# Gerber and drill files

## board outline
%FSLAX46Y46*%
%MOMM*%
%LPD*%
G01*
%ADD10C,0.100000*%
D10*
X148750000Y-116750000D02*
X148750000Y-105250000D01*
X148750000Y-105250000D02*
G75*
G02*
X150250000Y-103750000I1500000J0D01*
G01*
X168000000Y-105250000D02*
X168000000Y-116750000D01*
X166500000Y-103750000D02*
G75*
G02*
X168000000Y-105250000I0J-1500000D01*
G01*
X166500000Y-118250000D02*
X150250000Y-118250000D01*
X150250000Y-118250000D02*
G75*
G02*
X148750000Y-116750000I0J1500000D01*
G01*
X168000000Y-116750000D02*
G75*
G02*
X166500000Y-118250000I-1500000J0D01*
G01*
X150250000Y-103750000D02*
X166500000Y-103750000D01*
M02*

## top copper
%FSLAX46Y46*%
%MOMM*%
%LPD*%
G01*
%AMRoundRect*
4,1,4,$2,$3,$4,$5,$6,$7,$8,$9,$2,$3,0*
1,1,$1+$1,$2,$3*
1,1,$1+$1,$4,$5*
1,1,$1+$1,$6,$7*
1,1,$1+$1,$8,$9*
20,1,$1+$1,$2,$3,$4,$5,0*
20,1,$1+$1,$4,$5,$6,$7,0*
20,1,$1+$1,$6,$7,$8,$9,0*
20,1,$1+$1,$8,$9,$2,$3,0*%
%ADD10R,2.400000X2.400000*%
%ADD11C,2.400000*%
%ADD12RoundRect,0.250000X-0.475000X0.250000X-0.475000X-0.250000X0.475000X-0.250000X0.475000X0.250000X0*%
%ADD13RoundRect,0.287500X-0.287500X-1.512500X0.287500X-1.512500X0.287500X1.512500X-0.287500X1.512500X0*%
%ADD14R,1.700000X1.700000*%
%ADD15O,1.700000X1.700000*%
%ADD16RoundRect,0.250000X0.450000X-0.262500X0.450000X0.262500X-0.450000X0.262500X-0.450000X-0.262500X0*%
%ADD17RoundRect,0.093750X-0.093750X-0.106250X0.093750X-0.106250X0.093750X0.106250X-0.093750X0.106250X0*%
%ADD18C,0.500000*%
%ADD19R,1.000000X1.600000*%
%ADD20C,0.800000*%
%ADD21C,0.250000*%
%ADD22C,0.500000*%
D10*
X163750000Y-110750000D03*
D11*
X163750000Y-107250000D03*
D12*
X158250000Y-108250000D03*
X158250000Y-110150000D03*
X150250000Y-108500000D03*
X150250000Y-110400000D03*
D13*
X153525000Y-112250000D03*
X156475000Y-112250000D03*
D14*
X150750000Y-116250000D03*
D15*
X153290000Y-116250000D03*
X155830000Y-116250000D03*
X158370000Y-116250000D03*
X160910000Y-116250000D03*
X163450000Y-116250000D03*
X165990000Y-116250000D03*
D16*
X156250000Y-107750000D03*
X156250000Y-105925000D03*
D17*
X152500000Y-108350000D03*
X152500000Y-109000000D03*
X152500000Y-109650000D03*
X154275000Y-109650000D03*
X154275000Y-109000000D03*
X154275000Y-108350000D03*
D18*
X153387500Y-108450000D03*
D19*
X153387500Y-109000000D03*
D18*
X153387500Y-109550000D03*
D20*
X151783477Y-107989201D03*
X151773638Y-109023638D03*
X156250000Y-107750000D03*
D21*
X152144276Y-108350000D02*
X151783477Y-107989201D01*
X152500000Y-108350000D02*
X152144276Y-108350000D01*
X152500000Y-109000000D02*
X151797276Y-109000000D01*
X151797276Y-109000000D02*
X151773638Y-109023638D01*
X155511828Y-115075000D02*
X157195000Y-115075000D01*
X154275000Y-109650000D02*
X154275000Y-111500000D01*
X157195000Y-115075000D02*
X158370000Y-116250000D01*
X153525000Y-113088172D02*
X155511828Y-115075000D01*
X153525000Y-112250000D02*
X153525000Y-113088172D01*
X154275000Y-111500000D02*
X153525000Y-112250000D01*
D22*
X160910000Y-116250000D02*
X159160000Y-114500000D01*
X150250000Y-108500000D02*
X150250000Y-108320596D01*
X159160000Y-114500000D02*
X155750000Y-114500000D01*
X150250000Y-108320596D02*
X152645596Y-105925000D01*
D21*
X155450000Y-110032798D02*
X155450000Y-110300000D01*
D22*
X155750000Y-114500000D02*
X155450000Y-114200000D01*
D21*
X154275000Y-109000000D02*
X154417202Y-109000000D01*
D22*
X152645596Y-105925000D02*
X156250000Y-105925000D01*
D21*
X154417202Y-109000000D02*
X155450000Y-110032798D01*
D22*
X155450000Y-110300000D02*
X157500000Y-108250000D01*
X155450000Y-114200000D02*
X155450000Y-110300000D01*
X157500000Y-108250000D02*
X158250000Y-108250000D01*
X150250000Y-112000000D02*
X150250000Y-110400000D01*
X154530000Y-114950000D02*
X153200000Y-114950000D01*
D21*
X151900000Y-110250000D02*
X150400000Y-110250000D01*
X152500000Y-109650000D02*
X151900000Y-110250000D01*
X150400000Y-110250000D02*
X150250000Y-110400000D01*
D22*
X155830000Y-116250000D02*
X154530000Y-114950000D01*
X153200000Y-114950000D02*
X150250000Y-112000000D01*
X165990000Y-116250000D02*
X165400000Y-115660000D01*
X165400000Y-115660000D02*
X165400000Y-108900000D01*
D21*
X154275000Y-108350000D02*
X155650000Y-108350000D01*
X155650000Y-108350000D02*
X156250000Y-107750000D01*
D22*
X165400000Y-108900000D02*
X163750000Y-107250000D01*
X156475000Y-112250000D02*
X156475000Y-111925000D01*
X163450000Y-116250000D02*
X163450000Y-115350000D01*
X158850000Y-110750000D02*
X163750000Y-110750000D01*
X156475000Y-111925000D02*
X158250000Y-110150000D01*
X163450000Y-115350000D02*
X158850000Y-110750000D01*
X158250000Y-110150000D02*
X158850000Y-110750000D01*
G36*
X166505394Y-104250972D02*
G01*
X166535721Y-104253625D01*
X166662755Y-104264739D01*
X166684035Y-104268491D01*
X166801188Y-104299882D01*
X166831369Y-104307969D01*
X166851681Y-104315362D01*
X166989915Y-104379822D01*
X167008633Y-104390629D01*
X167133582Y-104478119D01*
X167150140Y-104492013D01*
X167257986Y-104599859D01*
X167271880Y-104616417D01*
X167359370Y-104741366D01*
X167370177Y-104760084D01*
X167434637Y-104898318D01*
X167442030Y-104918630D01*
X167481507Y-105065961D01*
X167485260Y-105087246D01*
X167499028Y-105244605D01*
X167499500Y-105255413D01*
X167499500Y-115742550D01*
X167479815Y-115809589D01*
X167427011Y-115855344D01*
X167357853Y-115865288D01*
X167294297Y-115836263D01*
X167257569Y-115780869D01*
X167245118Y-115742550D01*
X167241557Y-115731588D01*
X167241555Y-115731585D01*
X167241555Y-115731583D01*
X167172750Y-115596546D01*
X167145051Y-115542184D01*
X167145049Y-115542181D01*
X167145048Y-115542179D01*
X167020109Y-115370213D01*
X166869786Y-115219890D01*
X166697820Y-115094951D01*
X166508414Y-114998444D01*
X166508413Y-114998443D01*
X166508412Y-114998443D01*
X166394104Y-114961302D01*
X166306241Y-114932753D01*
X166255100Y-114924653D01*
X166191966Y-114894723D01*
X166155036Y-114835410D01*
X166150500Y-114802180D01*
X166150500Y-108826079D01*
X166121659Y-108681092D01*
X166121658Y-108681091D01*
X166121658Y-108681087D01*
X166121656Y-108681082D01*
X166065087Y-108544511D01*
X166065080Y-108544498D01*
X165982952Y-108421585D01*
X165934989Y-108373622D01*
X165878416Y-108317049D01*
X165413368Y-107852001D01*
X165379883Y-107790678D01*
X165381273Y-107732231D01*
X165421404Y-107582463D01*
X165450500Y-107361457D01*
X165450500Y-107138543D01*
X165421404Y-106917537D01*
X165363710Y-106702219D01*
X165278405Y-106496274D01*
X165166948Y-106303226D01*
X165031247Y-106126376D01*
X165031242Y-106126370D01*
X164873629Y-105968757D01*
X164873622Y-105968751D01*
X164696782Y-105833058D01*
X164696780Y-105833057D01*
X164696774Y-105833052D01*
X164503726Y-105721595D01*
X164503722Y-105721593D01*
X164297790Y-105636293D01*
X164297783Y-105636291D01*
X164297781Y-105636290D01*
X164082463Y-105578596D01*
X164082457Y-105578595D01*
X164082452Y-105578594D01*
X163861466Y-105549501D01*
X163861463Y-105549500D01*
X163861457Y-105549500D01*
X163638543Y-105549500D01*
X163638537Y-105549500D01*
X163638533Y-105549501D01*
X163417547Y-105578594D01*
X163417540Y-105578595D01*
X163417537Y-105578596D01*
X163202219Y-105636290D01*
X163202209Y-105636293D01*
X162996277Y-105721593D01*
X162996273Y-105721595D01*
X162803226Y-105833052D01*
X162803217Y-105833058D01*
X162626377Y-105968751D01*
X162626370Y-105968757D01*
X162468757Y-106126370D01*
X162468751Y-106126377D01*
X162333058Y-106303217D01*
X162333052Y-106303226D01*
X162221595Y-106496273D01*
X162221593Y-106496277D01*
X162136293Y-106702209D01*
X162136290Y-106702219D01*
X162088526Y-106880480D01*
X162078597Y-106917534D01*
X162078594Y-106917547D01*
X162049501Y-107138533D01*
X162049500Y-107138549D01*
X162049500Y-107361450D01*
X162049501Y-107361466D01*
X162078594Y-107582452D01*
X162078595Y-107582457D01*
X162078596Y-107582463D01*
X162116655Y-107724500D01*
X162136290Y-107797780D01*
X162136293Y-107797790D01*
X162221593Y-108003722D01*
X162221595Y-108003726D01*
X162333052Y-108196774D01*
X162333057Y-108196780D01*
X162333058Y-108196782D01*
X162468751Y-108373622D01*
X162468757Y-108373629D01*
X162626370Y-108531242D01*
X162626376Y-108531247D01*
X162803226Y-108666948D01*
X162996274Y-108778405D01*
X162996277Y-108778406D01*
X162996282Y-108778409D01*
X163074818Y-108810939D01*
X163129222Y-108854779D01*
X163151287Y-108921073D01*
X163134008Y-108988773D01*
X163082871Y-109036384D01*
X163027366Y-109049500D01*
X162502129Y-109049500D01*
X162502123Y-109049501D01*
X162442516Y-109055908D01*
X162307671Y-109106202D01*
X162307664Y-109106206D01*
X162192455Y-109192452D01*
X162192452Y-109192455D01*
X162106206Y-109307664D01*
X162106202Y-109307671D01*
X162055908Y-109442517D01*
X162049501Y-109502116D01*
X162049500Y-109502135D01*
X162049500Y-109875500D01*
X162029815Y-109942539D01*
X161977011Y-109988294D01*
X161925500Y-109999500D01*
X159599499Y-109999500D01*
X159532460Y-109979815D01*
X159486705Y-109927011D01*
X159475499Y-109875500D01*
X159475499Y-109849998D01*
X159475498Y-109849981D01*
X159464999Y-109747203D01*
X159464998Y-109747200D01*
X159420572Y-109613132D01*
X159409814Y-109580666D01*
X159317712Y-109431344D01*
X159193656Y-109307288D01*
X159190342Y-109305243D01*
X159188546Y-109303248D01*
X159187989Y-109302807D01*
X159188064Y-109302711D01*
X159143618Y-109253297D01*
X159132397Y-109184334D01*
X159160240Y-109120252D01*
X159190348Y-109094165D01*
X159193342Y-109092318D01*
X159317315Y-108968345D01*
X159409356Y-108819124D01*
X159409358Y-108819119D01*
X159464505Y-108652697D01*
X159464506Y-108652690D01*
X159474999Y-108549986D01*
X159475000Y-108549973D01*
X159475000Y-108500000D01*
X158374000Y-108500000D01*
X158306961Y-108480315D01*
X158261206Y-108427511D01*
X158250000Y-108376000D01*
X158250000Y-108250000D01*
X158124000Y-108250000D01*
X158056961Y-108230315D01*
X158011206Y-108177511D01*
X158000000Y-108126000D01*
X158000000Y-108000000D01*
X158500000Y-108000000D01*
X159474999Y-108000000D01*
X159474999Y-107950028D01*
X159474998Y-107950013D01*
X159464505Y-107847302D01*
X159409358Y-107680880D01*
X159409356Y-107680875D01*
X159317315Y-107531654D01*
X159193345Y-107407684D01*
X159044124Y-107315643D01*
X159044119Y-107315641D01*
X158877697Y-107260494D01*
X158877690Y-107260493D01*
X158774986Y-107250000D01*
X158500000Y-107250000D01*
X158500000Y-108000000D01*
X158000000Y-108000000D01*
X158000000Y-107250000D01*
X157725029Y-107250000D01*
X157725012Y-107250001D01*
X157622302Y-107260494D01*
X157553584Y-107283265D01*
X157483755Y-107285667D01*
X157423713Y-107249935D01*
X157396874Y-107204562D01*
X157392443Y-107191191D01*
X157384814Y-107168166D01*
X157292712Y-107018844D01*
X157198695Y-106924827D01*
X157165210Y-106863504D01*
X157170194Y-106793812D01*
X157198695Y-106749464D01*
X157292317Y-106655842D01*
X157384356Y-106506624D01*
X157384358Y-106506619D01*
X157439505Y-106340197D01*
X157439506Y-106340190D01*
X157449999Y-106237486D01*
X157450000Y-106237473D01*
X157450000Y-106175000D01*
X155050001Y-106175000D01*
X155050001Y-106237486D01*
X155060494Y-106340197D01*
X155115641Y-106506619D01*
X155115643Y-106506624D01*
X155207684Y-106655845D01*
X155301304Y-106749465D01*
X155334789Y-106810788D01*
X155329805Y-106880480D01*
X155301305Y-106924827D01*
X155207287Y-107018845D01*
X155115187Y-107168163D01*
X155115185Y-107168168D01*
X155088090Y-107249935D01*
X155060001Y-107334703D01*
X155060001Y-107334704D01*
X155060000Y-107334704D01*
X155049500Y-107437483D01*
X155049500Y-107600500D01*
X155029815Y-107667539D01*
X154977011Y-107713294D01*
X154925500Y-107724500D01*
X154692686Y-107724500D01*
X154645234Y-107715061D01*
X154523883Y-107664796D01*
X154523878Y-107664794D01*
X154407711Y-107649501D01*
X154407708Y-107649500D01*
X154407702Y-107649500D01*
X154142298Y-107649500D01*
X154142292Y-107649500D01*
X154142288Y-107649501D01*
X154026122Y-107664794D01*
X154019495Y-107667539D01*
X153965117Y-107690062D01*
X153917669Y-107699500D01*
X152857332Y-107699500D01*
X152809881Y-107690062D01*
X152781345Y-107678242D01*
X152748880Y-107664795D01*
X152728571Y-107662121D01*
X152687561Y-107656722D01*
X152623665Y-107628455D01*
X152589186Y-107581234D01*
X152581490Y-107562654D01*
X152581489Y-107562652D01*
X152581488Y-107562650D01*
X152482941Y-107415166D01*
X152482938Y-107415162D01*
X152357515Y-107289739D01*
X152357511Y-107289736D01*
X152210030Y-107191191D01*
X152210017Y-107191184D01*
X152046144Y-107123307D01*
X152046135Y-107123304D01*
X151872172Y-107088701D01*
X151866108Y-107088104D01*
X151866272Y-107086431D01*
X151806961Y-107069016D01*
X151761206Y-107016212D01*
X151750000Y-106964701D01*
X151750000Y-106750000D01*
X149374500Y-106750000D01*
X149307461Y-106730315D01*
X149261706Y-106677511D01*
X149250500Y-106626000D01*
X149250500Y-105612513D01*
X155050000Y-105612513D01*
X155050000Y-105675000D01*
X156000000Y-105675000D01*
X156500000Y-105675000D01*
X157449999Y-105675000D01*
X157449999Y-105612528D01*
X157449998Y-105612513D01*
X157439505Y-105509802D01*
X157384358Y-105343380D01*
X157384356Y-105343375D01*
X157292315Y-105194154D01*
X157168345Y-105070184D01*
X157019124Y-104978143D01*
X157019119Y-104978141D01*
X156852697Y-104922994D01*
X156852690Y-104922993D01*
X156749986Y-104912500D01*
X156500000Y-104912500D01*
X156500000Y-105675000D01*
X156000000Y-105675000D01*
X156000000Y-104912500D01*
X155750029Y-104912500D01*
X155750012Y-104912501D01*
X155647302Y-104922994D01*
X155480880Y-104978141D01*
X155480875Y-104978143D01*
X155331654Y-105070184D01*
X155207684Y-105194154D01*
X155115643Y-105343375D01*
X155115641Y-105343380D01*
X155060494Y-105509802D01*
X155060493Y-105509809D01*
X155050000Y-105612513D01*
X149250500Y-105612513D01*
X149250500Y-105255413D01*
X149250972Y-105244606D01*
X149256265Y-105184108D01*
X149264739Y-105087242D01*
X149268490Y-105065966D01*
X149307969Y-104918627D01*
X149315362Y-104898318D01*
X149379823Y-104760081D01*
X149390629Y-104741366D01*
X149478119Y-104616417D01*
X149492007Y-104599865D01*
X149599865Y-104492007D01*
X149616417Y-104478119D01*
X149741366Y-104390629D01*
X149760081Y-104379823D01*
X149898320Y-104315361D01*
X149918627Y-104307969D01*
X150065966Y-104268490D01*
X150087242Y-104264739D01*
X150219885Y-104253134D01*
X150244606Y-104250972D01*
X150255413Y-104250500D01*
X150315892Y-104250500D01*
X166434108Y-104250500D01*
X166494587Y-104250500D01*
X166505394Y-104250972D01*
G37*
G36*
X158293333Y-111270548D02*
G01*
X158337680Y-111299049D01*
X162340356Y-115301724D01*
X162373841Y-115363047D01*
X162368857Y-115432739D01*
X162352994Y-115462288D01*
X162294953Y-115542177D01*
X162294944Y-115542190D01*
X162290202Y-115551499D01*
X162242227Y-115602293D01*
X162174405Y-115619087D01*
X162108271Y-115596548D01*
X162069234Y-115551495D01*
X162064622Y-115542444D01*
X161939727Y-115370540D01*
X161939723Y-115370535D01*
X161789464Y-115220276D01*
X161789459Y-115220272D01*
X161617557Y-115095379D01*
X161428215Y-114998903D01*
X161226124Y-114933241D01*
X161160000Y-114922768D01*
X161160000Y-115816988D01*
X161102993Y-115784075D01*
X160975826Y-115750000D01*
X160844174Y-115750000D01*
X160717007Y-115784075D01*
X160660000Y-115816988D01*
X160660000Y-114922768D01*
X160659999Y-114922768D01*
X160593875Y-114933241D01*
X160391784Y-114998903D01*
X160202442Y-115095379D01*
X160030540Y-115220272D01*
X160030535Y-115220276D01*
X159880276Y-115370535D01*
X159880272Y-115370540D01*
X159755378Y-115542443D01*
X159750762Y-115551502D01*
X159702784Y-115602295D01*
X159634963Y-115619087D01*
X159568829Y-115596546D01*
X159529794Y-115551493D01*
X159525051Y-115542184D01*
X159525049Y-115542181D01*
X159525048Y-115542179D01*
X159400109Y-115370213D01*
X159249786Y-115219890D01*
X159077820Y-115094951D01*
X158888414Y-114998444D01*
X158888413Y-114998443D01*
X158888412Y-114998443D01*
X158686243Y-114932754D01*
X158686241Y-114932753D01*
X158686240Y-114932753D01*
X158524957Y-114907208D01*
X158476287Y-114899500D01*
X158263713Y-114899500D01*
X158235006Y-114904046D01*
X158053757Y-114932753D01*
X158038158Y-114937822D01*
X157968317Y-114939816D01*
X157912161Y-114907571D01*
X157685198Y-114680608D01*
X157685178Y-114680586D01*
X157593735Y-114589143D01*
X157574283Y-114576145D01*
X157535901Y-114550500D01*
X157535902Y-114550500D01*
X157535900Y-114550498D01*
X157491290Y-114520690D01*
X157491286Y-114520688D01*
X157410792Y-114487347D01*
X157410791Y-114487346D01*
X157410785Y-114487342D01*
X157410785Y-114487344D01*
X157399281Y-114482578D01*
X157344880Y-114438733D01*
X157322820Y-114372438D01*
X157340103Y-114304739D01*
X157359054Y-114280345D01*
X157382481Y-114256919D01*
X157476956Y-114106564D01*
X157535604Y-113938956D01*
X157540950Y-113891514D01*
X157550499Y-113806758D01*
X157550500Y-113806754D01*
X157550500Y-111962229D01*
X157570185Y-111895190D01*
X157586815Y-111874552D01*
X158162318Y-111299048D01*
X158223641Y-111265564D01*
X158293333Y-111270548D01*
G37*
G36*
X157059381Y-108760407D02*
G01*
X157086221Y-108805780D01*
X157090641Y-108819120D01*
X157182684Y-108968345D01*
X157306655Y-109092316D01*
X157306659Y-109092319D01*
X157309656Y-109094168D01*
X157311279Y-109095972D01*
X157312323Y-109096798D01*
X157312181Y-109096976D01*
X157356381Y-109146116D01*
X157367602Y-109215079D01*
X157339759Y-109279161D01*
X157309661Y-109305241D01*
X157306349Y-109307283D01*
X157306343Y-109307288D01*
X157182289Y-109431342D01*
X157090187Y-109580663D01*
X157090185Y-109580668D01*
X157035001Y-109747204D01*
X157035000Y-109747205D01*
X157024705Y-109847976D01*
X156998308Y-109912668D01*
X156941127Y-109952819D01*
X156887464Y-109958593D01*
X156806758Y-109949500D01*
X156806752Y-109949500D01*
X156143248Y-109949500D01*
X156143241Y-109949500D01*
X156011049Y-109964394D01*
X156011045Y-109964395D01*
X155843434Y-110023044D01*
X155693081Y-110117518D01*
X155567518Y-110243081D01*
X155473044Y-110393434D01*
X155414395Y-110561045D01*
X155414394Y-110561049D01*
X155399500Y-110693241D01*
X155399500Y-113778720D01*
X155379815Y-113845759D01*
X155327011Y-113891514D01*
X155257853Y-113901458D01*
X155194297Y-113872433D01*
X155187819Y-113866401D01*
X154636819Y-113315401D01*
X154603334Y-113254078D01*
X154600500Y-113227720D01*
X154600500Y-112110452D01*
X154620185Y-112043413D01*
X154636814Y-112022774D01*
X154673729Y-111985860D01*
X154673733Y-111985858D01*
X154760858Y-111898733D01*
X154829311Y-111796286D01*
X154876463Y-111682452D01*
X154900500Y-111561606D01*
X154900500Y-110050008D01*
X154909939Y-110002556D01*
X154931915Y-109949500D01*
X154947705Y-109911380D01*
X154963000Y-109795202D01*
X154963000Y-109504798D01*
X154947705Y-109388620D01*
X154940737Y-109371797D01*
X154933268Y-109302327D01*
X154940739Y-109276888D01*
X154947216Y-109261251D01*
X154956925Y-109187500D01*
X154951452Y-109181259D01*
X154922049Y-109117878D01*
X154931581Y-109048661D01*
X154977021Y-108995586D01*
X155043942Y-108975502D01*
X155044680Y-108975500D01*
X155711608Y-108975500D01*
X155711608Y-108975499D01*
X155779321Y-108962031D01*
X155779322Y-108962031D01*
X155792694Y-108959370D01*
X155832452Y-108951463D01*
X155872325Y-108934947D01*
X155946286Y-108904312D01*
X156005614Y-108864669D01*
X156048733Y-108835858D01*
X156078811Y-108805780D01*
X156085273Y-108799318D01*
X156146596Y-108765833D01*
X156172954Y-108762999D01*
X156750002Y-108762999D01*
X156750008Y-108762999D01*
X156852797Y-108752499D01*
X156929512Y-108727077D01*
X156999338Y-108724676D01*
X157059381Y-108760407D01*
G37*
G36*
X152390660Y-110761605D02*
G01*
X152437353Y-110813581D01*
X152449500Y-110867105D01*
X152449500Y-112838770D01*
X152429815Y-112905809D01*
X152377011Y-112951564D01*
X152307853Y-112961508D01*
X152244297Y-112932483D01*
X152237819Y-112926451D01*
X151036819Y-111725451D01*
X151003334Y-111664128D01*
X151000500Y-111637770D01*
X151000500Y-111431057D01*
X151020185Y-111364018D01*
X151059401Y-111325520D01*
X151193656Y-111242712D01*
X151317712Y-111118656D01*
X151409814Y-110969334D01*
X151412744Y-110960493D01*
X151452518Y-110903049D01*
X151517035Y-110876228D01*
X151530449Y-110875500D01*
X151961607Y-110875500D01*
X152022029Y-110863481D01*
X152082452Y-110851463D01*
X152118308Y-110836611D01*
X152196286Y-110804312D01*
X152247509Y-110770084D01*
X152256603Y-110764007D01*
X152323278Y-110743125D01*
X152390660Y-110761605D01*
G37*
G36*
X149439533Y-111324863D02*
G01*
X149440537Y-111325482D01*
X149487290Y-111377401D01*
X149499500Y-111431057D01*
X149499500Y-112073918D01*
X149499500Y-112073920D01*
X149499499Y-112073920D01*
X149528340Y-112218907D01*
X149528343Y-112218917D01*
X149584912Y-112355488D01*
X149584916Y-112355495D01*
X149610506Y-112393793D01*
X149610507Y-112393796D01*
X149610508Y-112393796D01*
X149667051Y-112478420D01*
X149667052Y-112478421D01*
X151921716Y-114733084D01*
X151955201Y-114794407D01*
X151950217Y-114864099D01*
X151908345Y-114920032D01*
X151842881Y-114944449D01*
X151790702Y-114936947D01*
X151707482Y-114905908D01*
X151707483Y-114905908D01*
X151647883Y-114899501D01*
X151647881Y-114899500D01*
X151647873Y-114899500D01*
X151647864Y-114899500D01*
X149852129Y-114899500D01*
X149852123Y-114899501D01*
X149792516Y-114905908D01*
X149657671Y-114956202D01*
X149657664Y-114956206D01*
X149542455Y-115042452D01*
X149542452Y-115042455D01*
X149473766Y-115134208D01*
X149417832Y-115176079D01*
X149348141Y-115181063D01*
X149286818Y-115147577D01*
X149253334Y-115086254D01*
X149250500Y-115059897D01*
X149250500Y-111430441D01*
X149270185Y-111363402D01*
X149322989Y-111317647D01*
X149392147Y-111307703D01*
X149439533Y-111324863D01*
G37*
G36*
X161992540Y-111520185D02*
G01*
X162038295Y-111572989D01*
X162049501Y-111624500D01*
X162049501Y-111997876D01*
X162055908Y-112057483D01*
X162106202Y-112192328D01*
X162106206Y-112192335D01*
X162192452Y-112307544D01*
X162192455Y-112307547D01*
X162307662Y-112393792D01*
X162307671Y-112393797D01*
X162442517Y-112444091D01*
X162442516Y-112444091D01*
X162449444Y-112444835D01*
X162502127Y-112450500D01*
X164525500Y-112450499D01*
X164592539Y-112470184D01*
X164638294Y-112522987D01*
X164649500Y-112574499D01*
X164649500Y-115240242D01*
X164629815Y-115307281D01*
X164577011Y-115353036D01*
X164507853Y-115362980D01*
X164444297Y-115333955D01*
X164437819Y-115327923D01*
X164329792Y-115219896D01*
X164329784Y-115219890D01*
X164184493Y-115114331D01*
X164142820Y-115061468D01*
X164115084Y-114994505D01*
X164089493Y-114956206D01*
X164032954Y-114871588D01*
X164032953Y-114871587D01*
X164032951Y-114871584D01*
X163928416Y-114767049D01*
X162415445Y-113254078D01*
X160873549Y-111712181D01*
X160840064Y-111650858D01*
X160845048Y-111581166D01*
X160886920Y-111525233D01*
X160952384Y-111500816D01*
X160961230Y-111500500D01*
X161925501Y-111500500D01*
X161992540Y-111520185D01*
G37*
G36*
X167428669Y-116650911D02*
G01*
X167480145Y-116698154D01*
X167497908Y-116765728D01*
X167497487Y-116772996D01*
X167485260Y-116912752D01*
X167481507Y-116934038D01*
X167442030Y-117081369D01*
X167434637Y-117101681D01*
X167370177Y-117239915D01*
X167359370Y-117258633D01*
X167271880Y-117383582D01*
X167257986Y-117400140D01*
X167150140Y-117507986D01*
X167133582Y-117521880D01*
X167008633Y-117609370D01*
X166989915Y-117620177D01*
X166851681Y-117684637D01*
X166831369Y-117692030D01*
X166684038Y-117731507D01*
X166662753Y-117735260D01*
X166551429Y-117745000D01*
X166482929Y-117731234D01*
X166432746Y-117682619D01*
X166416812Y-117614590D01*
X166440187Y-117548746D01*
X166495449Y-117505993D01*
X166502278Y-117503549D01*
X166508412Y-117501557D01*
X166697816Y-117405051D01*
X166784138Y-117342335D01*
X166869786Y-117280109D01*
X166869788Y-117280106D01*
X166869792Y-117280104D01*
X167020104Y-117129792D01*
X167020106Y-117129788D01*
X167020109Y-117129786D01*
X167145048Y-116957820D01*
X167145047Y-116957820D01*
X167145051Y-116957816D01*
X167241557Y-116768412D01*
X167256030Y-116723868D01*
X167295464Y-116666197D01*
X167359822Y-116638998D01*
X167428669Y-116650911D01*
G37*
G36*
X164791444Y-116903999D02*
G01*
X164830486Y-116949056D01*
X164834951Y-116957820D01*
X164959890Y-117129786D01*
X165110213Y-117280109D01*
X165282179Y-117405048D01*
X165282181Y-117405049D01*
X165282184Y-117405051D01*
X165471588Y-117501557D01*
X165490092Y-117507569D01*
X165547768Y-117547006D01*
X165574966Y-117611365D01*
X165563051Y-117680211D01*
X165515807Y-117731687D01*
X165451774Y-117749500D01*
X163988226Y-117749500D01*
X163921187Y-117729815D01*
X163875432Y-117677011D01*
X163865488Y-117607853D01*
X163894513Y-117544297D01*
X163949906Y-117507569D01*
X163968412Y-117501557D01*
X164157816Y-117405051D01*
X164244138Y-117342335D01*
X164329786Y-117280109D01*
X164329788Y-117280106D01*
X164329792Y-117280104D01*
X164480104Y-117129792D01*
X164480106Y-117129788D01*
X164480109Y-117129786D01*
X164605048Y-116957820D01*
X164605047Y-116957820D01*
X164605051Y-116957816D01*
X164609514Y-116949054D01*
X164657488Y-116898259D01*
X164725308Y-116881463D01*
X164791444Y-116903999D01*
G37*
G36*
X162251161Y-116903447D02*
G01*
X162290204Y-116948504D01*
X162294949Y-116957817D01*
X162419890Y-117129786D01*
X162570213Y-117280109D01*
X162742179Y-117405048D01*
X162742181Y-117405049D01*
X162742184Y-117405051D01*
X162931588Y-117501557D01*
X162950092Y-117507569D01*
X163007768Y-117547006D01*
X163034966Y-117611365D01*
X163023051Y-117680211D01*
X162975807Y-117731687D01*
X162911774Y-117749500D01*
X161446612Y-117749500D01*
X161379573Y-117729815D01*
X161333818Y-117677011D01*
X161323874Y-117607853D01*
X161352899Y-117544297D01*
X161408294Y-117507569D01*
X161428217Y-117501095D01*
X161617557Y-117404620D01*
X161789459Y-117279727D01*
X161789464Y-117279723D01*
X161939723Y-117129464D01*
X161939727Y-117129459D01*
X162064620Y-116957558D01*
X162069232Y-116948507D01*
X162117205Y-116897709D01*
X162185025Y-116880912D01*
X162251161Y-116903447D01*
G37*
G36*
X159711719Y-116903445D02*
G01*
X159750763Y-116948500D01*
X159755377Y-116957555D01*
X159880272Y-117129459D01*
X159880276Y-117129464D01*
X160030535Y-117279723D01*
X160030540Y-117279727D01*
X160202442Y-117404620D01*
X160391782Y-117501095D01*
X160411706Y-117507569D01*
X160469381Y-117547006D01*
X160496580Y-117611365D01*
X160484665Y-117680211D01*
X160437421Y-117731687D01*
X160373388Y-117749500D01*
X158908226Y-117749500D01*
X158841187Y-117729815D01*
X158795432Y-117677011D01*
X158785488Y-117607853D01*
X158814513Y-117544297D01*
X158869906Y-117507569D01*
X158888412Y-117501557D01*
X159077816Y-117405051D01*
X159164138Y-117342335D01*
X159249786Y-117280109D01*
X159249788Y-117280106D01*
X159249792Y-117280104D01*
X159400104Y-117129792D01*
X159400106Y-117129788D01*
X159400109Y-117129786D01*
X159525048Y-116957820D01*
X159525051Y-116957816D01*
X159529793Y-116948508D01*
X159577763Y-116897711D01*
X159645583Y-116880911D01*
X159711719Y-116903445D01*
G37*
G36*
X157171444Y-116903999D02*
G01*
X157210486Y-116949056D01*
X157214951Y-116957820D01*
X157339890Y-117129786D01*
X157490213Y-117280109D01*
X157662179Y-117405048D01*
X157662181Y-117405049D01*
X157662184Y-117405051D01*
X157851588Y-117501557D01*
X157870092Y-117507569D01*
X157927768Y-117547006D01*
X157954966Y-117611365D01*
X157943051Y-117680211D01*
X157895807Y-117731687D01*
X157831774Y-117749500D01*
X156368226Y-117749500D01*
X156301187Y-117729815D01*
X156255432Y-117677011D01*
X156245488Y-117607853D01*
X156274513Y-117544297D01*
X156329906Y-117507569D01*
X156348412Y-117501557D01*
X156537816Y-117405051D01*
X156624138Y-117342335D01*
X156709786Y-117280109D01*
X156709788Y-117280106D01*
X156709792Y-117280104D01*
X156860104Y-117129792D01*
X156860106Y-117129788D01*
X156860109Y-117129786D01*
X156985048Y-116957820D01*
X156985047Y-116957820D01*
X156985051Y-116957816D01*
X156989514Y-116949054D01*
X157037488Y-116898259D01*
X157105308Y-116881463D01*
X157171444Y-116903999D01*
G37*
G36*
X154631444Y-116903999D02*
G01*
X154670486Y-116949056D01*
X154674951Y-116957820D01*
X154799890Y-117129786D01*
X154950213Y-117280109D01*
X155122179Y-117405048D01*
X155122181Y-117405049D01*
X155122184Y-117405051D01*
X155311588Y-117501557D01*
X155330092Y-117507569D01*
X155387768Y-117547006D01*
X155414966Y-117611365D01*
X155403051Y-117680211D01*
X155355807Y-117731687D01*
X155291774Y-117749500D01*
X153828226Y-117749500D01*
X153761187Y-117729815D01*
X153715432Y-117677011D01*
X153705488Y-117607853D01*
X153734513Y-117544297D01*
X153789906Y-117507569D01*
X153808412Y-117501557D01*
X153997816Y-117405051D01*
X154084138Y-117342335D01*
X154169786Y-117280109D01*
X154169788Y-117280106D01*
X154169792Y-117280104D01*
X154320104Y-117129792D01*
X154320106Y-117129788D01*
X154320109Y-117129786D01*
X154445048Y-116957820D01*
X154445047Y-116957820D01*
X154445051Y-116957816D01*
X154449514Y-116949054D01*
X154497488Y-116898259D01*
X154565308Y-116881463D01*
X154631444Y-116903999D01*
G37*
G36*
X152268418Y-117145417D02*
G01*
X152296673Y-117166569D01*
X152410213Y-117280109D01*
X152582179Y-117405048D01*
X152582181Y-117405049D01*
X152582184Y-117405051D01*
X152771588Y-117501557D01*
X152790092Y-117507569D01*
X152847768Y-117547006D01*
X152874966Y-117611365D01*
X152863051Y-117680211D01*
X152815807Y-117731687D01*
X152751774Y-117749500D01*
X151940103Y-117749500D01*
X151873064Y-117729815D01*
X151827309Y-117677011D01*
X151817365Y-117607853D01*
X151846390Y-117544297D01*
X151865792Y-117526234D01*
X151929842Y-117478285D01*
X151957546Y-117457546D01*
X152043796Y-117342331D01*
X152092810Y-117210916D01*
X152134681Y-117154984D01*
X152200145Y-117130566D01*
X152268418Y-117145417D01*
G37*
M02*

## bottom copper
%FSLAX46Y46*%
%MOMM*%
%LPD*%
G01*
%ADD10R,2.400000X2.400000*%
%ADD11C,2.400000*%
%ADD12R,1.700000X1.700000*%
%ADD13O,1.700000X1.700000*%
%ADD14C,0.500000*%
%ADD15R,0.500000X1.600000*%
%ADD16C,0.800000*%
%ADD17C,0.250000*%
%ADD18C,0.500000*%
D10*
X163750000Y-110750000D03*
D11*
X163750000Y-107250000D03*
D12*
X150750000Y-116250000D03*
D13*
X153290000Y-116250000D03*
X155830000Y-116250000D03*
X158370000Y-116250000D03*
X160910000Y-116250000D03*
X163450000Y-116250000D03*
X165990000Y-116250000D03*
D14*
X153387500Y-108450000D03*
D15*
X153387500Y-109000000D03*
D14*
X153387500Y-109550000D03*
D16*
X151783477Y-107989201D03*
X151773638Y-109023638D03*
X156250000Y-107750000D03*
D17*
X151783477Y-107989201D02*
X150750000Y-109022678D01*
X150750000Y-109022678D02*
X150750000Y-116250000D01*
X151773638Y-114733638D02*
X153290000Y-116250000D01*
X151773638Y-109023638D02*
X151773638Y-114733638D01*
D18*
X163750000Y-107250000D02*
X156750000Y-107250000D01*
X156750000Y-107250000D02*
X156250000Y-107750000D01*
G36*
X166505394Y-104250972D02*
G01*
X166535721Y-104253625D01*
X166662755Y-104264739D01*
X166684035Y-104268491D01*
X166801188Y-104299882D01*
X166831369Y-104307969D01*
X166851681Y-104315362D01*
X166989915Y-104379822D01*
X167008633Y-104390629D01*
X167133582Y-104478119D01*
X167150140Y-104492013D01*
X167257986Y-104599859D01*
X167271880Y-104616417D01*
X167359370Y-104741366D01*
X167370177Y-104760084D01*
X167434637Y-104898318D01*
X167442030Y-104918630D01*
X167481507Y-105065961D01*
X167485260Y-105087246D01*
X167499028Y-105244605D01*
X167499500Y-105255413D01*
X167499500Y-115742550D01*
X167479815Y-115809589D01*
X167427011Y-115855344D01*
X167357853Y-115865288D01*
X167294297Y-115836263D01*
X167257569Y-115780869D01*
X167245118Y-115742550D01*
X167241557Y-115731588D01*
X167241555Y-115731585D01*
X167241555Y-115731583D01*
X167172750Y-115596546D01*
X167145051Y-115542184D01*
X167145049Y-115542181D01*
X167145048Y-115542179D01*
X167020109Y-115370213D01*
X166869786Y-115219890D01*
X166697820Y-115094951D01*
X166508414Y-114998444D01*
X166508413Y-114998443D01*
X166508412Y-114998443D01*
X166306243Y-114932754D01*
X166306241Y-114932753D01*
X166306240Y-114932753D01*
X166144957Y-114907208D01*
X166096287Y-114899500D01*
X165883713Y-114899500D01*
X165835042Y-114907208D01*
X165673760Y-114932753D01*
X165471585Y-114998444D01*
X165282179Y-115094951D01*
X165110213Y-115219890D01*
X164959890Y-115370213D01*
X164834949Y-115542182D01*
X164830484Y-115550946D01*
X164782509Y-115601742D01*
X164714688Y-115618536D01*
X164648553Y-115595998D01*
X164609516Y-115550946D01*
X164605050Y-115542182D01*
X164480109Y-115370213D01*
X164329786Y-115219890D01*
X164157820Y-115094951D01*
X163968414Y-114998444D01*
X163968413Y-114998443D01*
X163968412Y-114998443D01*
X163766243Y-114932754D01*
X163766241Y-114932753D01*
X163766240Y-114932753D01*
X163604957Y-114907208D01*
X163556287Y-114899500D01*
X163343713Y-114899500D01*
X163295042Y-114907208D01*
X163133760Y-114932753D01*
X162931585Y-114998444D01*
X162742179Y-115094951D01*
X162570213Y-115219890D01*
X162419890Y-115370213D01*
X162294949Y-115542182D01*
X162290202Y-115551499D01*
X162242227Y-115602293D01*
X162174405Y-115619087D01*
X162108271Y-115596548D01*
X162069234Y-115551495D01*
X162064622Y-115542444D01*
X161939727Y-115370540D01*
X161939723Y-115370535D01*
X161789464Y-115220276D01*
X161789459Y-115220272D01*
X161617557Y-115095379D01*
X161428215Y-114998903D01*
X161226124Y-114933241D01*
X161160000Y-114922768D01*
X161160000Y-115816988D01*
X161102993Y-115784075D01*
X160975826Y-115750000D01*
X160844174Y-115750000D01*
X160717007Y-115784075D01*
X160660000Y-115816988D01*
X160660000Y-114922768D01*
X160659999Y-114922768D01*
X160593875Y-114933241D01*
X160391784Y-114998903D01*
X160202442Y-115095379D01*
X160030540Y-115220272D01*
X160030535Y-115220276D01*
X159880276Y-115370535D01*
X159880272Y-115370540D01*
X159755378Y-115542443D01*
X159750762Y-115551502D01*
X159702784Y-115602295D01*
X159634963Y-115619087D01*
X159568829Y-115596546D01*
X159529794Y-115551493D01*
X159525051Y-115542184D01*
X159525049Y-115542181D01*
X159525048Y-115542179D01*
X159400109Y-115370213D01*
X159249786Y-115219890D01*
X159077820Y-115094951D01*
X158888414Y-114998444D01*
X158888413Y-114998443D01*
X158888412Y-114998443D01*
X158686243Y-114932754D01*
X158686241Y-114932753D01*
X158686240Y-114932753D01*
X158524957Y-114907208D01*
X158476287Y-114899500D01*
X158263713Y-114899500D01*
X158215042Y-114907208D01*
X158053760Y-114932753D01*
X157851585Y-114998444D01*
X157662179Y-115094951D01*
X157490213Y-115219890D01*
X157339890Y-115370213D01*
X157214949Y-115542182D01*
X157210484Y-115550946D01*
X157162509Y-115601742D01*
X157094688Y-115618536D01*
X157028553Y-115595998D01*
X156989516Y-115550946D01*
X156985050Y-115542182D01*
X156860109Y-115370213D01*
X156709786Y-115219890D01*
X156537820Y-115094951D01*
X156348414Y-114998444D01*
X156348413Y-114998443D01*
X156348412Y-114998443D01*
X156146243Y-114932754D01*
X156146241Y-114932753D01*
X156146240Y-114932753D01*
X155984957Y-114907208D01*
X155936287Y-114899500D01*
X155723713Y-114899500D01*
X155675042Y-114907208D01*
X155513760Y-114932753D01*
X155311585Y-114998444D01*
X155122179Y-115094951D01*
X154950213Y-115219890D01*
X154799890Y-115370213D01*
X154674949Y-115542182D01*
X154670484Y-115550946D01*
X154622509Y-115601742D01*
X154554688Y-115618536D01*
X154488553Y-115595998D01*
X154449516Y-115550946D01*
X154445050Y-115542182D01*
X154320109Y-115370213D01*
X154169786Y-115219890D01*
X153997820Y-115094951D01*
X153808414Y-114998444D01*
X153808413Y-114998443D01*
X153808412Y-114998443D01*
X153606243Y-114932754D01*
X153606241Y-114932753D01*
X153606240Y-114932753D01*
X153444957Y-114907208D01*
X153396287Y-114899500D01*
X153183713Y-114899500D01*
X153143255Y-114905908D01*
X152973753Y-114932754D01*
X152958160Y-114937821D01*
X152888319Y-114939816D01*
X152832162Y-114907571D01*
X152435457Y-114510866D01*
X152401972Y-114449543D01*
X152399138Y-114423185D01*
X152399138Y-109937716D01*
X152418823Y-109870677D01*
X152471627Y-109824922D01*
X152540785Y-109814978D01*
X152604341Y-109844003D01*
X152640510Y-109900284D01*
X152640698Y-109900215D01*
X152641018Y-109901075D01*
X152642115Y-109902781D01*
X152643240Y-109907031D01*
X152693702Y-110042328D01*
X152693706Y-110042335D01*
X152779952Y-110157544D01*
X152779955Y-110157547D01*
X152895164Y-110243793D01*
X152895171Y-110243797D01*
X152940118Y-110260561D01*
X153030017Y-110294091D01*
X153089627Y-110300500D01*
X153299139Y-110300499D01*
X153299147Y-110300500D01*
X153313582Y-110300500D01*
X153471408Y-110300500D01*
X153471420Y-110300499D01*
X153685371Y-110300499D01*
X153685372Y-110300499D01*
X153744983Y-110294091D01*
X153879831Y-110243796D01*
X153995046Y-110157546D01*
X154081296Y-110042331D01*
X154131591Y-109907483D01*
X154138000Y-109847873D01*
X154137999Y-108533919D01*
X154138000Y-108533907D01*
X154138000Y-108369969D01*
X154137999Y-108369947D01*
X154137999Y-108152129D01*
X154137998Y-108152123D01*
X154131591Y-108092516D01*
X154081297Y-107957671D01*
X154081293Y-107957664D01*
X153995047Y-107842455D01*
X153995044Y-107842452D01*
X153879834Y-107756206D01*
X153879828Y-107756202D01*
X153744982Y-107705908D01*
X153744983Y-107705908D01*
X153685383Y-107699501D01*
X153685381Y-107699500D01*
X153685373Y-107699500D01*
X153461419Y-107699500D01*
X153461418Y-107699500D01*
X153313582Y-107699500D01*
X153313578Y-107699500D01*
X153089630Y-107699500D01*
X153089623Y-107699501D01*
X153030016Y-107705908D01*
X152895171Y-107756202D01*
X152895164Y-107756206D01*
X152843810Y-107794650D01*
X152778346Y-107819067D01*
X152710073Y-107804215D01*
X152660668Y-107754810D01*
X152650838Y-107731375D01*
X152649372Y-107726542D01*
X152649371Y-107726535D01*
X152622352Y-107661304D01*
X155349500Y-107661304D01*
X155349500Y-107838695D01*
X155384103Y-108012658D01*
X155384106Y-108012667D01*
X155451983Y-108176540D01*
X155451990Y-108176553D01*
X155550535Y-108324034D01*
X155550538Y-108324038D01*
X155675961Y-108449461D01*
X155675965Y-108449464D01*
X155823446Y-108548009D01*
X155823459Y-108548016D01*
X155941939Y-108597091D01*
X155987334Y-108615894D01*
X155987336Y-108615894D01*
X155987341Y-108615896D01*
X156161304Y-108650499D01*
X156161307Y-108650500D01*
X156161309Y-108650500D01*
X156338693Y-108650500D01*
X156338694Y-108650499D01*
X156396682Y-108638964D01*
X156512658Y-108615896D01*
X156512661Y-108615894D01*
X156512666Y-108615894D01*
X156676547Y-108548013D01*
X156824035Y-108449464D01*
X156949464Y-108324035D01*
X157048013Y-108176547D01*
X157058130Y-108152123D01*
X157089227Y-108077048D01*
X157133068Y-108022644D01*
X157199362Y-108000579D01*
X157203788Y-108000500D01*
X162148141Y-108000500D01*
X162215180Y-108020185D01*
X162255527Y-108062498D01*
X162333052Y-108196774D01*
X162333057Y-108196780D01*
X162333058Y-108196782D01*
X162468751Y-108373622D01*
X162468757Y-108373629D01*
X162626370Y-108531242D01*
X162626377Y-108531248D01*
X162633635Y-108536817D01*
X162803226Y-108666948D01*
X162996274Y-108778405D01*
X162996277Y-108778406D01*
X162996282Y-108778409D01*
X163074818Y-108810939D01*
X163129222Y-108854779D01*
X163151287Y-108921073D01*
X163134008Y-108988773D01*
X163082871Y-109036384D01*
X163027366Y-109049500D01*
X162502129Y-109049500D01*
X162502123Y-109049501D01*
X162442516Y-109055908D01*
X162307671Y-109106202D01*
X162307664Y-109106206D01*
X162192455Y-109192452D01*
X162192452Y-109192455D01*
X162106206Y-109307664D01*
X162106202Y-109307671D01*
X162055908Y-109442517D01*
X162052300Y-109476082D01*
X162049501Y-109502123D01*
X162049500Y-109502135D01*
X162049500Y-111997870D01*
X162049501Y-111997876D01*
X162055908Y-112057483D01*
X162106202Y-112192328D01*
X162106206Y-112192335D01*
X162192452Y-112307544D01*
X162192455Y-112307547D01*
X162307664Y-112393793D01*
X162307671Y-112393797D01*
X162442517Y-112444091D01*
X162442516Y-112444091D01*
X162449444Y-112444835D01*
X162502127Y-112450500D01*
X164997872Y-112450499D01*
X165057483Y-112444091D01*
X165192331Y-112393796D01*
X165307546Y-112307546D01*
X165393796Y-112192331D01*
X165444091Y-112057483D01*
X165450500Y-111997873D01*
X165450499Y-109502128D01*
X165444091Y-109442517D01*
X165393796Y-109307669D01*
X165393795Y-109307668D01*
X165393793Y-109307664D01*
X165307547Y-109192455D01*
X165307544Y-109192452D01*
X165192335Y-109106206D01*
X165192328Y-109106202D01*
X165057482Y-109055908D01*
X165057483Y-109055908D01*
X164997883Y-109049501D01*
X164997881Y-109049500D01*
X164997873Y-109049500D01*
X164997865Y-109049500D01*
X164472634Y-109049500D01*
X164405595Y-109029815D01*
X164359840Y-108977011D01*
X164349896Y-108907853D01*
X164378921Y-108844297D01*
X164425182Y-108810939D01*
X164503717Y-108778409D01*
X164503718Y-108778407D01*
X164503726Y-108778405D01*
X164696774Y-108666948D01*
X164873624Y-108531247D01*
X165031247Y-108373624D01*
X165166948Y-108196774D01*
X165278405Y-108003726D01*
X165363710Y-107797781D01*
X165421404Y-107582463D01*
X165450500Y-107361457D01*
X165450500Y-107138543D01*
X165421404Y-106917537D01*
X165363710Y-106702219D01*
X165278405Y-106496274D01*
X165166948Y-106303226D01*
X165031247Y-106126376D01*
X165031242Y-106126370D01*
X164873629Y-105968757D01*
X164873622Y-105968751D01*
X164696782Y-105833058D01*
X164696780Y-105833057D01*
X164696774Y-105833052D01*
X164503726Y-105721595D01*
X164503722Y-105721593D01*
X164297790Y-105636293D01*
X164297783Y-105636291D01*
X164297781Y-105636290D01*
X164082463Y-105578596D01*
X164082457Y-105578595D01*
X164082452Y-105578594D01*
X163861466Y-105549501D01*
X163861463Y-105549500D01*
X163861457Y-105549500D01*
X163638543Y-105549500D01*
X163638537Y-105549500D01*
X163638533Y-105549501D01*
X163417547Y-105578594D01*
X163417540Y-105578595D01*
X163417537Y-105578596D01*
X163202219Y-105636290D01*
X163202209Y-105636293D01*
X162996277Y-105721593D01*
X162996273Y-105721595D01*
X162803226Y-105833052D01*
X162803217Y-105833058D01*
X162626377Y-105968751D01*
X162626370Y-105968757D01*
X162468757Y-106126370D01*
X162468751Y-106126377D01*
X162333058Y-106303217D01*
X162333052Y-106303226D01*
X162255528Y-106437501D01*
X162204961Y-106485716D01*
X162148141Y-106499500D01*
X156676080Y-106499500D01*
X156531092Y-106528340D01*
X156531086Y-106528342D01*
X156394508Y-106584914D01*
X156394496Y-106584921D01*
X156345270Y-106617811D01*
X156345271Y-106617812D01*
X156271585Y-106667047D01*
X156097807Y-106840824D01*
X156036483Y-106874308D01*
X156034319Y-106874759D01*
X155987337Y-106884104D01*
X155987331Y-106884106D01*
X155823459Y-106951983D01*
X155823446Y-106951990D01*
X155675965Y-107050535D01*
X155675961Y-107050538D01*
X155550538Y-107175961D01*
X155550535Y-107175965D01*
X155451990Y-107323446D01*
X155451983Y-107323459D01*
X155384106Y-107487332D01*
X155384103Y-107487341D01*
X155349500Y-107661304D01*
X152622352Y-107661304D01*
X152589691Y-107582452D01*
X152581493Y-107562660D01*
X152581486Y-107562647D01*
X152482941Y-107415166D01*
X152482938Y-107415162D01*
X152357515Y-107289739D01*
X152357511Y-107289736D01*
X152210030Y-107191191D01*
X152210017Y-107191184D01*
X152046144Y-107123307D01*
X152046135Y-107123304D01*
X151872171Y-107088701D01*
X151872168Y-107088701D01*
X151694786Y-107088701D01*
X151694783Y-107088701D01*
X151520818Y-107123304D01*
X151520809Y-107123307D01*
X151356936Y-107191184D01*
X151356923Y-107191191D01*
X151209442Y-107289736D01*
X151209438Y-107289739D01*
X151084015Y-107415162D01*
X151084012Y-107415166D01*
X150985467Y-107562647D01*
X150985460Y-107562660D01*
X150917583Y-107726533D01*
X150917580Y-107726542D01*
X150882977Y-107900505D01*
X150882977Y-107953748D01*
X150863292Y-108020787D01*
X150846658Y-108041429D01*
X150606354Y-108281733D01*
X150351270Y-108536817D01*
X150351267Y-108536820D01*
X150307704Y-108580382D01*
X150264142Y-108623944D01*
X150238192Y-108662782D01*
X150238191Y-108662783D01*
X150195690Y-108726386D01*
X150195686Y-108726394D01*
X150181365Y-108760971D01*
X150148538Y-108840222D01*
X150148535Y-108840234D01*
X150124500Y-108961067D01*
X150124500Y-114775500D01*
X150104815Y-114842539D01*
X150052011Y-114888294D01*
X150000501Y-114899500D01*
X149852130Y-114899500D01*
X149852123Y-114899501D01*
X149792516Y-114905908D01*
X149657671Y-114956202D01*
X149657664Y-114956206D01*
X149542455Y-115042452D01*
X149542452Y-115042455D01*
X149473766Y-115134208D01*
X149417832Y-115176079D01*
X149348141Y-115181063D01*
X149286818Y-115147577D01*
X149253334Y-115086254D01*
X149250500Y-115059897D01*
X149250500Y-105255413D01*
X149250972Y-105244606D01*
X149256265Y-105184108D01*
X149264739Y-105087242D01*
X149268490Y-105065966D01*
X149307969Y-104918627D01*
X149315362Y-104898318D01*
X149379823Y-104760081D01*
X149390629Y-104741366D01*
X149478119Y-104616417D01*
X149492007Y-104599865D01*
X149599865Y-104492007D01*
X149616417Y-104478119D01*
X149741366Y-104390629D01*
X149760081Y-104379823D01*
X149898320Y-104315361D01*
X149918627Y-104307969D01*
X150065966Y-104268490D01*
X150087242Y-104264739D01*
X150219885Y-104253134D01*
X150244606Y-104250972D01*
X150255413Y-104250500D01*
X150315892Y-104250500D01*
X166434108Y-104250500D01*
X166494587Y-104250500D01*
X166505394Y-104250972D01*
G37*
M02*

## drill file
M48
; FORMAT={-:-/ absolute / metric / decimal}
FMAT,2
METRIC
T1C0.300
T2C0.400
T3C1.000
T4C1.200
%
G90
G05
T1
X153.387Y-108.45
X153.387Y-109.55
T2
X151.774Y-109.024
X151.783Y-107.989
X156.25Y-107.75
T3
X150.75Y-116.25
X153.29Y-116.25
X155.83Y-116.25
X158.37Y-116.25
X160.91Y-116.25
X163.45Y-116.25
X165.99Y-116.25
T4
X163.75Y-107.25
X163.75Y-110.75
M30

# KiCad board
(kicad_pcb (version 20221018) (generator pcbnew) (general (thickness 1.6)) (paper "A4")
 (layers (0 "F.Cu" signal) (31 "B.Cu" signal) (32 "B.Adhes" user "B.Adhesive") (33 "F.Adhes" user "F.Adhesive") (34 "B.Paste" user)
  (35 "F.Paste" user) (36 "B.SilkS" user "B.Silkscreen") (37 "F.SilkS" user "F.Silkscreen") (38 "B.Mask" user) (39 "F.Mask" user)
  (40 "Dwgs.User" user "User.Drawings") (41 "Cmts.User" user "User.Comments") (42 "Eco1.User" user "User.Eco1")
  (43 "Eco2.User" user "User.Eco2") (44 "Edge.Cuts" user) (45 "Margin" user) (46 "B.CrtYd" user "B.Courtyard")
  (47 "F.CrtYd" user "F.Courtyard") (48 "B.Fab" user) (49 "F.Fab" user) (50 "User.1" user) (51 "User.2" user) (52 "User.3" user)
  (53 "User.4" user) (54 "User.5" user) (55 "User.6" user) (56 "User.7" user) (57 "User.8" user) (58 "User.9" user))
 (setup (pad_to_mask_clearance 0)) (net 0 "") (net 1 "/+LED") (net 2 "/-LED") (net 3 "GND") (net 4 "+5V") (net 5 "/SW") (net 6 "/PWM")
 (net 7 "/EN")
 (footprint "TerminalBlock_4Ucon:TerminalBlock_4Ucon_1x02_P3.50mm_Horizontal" (layer "F.Cu") (at 163.75 110.75 90)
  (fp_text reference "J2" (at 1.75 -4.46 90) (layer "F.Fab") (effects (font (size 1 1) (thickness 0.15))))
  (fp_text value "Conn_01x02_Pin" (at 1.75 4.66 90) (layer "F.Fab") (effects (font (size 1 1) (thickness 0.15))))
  (pad "1" thru_hole rect (at 0 0 90) (size 2.4 2.4) (drill 1.2) (layers "*.Cu" "*.Mask") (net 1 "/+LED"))
  (pad "2" thru_hole circle (at 3.5 0 90) (size 2.4 2.4) (drill 1.2) (layers "*.Cu" "*.Mask") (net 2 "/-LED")))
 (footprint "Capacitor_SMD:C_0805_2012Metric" (layer "F.Cu") (at 158.25 109.2 -90)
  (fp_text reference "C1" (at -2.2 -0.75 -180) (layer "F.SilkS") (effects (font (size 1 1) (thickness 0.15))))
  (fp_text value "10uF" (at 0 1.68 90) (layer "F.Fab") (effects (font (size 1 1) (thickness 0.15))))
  (pad "1" smd roundrect (at -0.95 0 270) (size 1 1.45) (layers "F.Cu" "F.Paste" "F.Mask") (roundrect_rratio 0.25) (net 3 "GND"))
  (pad "2" smd roundrect (at 0.95 0 270) (size 1 1.45) (layers "F.Cu" "F.Paste" "F.Mask") (roundrect_rratio 0.25) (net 1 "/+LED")))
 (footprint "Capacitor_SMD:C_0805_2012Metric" (layer "F.Cu") (at 150.25 109.45 -90)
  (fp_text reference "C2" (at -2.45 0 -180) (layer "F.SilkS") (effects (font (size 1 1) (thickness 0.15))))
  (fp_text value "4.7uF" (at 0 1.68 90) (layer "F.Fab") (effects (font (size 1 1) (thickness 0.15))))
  (pad "1" smd roundrect (at -0.95 0 270) (size 1 1.45) (layers "F.Cu" "F.Paste" "F.Mask") (roundrect_rratio 0.25) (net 3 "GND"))
  (pad "2" smd roundrect (at 0.95 0 270) (size 1 1.45) (layers "F.Cu" "F.Paste" "F.Mask") (roundrect_rratio 0.25) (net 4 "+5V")))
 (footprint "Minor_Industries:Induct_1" (layer "F.Cu") (at 155 112.25)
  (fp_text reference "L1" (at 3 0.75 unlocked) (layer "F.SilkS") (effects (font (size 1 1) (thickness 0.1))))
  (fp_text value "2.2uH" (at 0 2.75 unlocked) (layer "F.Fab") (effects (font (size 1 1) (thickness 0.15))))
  (pad "1" smd roundrect (at -1.475 0) (size 1.15 3.6) (layers "F.Cu" "F.Paste" "F.Mask") (roundrect_rratio 0.25) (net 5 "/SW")
   (thermal_bridge_angle 45))
  (pad "2" smd roundrect (at 1.475 0) (size 1.15 3.6) (layers "F.Cu" "F.Paste" "F.Mask") (roundrect_rratio 0.25) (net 1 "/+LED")
   (thermal_bridge_angle 45)))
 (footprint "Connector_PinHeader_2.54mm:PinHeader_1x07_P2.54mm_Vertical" (layer "F.Cu") (at 150.75 116.25 90)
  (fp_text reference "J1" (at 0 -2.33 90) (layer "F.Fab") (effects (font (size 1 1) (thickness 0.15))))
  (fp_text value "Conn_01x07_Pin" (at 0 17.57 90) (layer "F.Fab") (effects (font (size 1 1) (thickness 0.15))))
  (pad "1" thru_hole rect (at 0 0 90) (size 1.7 1.7) (drill 1) (layers "*.Cu" "*.Mask") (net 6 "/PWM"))
  (pad "2" thru_hole oval (at 0 2.54 90) (size 1.7 1.7) (drill 1) (layers "*.Cu" "*.Mask") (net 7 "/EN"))
  (pad "3" thru_hole oval (at 0 5.08 90) (size 1.7 1.7) (drill 1) (layers "*.Cu" "*.Mask") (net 4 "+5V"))
  (pad "4" thru_hole oval (at 0 7.62 90) (size 1.7 1.7) (drill 1) (layers "*.Cu" "*.Mask") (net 5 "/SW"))
  (pad "5" thru_hole oval (at 0 10.16 90) (size 1.7 1.7) (drill 1) (layers "*.Cu" "*.Mask") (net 3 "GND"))
  (pad "6" thru_hole oval (at 0 12.7 90) (size 1.7 1.7) (drill 1) (layers "*.Cu" "*.Mask") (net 1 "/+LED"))
  (pad "7" thru_hole oval (at 0 15.24 90) (size 1.7 1.7) (drill 1) (layers "*.Cu" "*.Mask") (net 2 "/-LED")))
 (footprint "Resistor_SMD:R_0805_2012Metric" (layer "F.Cu") (at 156.25 106.8375 90)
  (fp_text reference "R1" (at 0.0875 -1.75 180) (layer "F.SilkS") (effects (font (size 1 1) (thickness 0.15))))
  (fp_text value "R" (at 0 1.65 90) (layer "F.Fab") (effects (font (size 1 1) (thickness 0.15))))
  (pad "1" smd roundrect (at -0.9125 0 90) (size 1.025 1.4) (layers "F.Cu" "F.Paste" "F.Mask") (roundrect_rratio 0.243902) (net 2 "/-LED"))
  (pad "2" smd roundrect (at 0.9125 0 90) (size 1.025 1.4) (layers "F.Cu" "F.Paste" "F.Mask") (roundrect_rratio 0.243902) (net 3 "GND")))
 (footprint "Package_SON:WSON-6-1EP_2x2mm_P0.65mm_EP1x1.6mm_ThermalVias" (layer "F.Cu") (at 153.3875 109)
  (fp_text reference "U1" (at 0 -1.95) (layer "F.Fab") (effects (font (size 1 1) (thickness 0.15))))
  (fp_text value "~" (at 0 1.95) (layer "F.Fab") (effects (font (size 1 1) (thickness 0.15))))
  (pad "" smd roundrect (at 0 -0.4) (size 0.87 0.69) (layers "F.Paste") (roundrect_rratio 0.25))
  (pad "" smd roundrect (at 0 0.4) (size 0.87 0.69) (layers "F.Paste") (roundrect_rratio 0.25))
  (pad "1" smd roundrect (at -0.8875 -0.65) (size 0.375 0.4) (layers "F.Cu" "F.Paste" "F.Mask") (roundrect_rratio 0.25) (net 6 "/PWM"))
  (pad "2" smd roundrect (at -0.8875 0) (size 0.375 0.4) (layers "F.Cu" "F.Paste" "F.Mask") (roundrect_rratio 0.25) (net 7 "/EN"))
  (pad "3" smd roundrect (at -0.8875 0.65) (size 0.375 0.4) (layers "F.Cu" "F.Paste" "F.Mask") (roundrect_rratio 0.25) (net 4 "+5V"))
  (pad "4" smd roundrect (at 0.8875 0.65) (size 0.375 0.4) (layers "F.Cu" "F.Paste" "F.Mask") (roundrect_rratio 0.25) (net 5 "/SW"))
  (pad "5" smd roundrect (at 0.8875 0) (size 0.375 0.4) (layers "F.Cu" "F.Paste" "F.Mask") (roundrect_rratio 0.25) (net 3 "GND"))
  (pad "6" smd roundrect (at 0.8875 -0.65) (size 0.375 0.4) (layers "F.Cu" "F.Paste" "F.Mask") (roundrect_rratio 0.25) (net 2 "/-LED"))
  (pad "7" thru_hole circle (at 0 -0.55) (size 0.5 0.5) (drill 0.3) (layers "*.Cu"))
  (pad "7" smd rect (at 0 0) (size 0.5 1.6) (layers "B.Cu"))
  (pad "7" smd rect (at 0 0) (size 1 1.6) (layers "F.Cu" "F.Mask"))
  (pad "7" thru_hole circle (at 0 0.55) (size 0.5 0.5) (drill 0.3) (layers "*.Cu")))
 (gr_line (start 148.75 116.75) (end 148.75 105.25) (stroke (width 0.1) (type default)) (layer "Edge.Cuts"))
 (gr_arc (start 148.75 105.25) (mid 149.18934 104.18934) (end 150.25 103.75) (stroke (width 0.1) (type default)) (layer "Edge.Cuts"))
 (gr_line (start 168 105.25) (end 168 116.75) (stroke (width 0.1) (type default)) (layer "Edge.Cuts"))
 (gr_arc (start 166.5 103.75) (mid 167.56066 104.18934) (end 168 105.25) (stroke (width 0.1) (type default)) (layer "Edge.Cuts"))
 (gr_line (start 166.5 118.25) (end 150.25 118.25) (stroke (width 0.1) (type default)) (layer "Edge.Cuts"))
 (gr_arc (start 150.25 118.25) (mid 149.18934 117.81066) (end 148.75 116.75) (stroke (width 0.1) (type default)) (layer "Edge.Cuts"))
 (gr_arc (start 168 116.75) (mid 167.56066 117.81066) (end 166.5 118.25) (stroke (width 0.1) (type default)) (layer "Edge.Cuts"))
 (gr_line (start 150.25 103.75) (end 166.5 103.75) (stroke (width 0.1) (type default)) (layer "Edge.Cuts"))
 (segment (start 152.144276 108.35) (end 151.783477 107.989201) (width 0.25) (layer "F.Cu") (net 6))
 (segment (start 152.5 108.35) (end 152.144276 108.35) (width 0.25) (layer "F.Cu") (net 6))
 (via (at 151.783477 107.989201) (size 0.8) (drill 0.4) (layers "F.Cu" "B.Cu") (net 6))
 (segment (start 151.783477 107.989201) (end 150.75 109.022678) (width 0.25) (layer "B.Cu") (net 6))
 (segment (start 150.75 109.022678) (end 150.75 116.25) (width 0.25) (layer "B.Cu") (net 6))
 (segment (start 152.5 109) (end 151.797276 109) (width 0.25) (layer "F.Cu") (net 7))
 (segment (start 151.797276 109) (end 151.773638 109.023638) (width 0.25) (layer "F.Cu") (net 7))
 (via (at 151.773638 109.023638) (size 0.8) (drill 0.4) (layers "F.Cu" "B.Cu") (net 7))
 (segment (start 151.773638 114.733638) (end 153.29 116.25) (width 0.25) (layer "B.Cu") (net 7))
 (segment (start 151.773638 109.023638) (end 151.773638 114.733638) (width 0.25) (layer "B.Cu") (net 7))
 (segment (start 155.511828 115.075) (end 157.195 115.075) (width 0.25) (layer "F.Cu") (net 5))
 (segment (start 154.275 109.65) (end 154.275 111.5) (width 0.25) (layer "F.Cu") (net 5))
 (segment (start 157.195 115.075) (end 158.37 116.25) (width 0.25) (layer "F.Cu") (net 5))
 (segment (start 153.525 113.088172) (end 155.511828 115.075) (width 0.25) (layer "F.Cu") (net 5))
 (segment (start 153.525 112.25) (end 153.525 113.088172) (width 0.25) (layer "F.Cu") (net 5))
 (segment (start 154.275 111.5) (end 153.525 112.25) (width 0.25) (layer "F.Cu") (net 5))
 (segment (start 160.91 116.25) (end 159.16 114.5) (width 0.5) (layer "F.Cu") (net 3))
 (segment (start 150.25 108.5) (end 150.25 108.320596) (width 0.5) (layer "F.Cu") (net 3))
 (segment (start 159.16 114.5) (end 155.75 114.5) (width 0.5) (layer "F.Cu") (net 3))
 (segment (start 150.25 108.320596) (end 152.645596 105.925) (width 0.5) (layer "F.Cu") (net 3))
 (segment (start 155.45 110.032798) (end 155.45 110.3) (width 0.25) (layer "F.Cu") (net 3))
 (segment (start 155.75 114.5) (end 155.45 114.2) (width 0.5) (layer "F.Cu") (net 3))
 (segment (start 154.275 109) (end 154.417202 109) (width 0.25) (layer "F.Cu") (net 3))
 (segment (start 152.645596 105.925) (end 156.25 105.925) (width 0.5) (layer "F.Cu") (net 3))
 (segment (start 154.417202 109) (end 155.45 110.032798) (width 0.25) (layer "F.Cu") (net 3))
 (segment (start 155.45 110.3) (end 157.5 108.25) (width 0.5) (layer "F.Cu") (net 3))
 (segment (start 155.45 114.2) (end 155.45 110.3) (width 0.5) (layer "F.Cu") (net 3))
 (segment (start 157.5 108.25) (end 158.25 108.25) (width 0.5) (layer "F.Cu") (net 3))
 (segment (start 150.25 112) (end 150.25 110.4) (width 0.5) (layer "F.Cu") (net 4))
 (segment (start 154.53 114.95) (end 153.2 114.95) (width 0.5) (layer "F.Cu") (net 4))
 (segment (start 151.9 110.25) (end 150.4 110.25) (width 0.25) (layer "F.Cu") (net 4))
 (segment (start 152.5 109.65) (end 151.9 110.25) (width 0.25) (layer "F.Cu") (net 4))
 (segment (start 150.4 110.25) (end 150.25 110.4) (width 0.25) (layer "F.Cu") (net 4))
 (segment (start 155.83 116.25) (end 154.53 114.95) (width 0.5) (layer "F.Cu") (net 4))
 (segment (start 153.2 114.95) (end 150.25 112) (width 0.5) (layer "F.Cu") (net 4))
 (segment (start 165.99 116.25) (end 165.4 115.66) (width 0.5) (layer "F.Cu") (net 2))
 (segment (start 165.4 115.66) (end 165.4 108.9) (width 0.5) (layer "F.Cu") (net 2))
 (segment (start 154.275 108.35) (end 155.65 108.35) (width 0.25) (layer "F.Cu") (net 2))
 (segment (start 155.65 108.35) (end 156.25 107.75) (width 0.25) (layer "F.Cu") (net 2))
 (segment (start 165.4 108.9) (end 163.75 107.25) (width 0.5) (layer "F.Cu") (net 2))
 (via (at 156.25 107.75) (size 0.8) (drill 0.4) (layers "F.Cu" "B.Cu") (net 2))
 (segment (start 163.75 107.25) (end 156.75 107.25) (width 0.5) (layer "B.Cu") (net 2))
 (segment (start 156.75 107.25) (end 156.25 107.75) (width 0.5) (layer "B.Cu") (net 2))
 (segment (start 156.475 112.25) (end 156.475 111.925) (width 0.5) (layer "F.Cu") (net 1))
 (segment (start 163.45 116.25) (end 163.45 115.35) (width 0.5) (layer "F.Cu") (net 1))
 (segment (start 158.85 110.75) (end 163.75 110.75) (width 0.5) (layer "F.Cu") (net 1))
 (segment (start 156.475 111.925) (end 158.25 110.15) (width 0.5) (layer "F.Cu") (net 1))
 (segment (start 163.45 115.35) (end 158.85 110.75) (width 0.5) (layer "F.Cu") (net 1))
 (segment (start 158.25 110.15) (end 158.85 110.75) (width 0.5) (layer "F.Cu") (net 1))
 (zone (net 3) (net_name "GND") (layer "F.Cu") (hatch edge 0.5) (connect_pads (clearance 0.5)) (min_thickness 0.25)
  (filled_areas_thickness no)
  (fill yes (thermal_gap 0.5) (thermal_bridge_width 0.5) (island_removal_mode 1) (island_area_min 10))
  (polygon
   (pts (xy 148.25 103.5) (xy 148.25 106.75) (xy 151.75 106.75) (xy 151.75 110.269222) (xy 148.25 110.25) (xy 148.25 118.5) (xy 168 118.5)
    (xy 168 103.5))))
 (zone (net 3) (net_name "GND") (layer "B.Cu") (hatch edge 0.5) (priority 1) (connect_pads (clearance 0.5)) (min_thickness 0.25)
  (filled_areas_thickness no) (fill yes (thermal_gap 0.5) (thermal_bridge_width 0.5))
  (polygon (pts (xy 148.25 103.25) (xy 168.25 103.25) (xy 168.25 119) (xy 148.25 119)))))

